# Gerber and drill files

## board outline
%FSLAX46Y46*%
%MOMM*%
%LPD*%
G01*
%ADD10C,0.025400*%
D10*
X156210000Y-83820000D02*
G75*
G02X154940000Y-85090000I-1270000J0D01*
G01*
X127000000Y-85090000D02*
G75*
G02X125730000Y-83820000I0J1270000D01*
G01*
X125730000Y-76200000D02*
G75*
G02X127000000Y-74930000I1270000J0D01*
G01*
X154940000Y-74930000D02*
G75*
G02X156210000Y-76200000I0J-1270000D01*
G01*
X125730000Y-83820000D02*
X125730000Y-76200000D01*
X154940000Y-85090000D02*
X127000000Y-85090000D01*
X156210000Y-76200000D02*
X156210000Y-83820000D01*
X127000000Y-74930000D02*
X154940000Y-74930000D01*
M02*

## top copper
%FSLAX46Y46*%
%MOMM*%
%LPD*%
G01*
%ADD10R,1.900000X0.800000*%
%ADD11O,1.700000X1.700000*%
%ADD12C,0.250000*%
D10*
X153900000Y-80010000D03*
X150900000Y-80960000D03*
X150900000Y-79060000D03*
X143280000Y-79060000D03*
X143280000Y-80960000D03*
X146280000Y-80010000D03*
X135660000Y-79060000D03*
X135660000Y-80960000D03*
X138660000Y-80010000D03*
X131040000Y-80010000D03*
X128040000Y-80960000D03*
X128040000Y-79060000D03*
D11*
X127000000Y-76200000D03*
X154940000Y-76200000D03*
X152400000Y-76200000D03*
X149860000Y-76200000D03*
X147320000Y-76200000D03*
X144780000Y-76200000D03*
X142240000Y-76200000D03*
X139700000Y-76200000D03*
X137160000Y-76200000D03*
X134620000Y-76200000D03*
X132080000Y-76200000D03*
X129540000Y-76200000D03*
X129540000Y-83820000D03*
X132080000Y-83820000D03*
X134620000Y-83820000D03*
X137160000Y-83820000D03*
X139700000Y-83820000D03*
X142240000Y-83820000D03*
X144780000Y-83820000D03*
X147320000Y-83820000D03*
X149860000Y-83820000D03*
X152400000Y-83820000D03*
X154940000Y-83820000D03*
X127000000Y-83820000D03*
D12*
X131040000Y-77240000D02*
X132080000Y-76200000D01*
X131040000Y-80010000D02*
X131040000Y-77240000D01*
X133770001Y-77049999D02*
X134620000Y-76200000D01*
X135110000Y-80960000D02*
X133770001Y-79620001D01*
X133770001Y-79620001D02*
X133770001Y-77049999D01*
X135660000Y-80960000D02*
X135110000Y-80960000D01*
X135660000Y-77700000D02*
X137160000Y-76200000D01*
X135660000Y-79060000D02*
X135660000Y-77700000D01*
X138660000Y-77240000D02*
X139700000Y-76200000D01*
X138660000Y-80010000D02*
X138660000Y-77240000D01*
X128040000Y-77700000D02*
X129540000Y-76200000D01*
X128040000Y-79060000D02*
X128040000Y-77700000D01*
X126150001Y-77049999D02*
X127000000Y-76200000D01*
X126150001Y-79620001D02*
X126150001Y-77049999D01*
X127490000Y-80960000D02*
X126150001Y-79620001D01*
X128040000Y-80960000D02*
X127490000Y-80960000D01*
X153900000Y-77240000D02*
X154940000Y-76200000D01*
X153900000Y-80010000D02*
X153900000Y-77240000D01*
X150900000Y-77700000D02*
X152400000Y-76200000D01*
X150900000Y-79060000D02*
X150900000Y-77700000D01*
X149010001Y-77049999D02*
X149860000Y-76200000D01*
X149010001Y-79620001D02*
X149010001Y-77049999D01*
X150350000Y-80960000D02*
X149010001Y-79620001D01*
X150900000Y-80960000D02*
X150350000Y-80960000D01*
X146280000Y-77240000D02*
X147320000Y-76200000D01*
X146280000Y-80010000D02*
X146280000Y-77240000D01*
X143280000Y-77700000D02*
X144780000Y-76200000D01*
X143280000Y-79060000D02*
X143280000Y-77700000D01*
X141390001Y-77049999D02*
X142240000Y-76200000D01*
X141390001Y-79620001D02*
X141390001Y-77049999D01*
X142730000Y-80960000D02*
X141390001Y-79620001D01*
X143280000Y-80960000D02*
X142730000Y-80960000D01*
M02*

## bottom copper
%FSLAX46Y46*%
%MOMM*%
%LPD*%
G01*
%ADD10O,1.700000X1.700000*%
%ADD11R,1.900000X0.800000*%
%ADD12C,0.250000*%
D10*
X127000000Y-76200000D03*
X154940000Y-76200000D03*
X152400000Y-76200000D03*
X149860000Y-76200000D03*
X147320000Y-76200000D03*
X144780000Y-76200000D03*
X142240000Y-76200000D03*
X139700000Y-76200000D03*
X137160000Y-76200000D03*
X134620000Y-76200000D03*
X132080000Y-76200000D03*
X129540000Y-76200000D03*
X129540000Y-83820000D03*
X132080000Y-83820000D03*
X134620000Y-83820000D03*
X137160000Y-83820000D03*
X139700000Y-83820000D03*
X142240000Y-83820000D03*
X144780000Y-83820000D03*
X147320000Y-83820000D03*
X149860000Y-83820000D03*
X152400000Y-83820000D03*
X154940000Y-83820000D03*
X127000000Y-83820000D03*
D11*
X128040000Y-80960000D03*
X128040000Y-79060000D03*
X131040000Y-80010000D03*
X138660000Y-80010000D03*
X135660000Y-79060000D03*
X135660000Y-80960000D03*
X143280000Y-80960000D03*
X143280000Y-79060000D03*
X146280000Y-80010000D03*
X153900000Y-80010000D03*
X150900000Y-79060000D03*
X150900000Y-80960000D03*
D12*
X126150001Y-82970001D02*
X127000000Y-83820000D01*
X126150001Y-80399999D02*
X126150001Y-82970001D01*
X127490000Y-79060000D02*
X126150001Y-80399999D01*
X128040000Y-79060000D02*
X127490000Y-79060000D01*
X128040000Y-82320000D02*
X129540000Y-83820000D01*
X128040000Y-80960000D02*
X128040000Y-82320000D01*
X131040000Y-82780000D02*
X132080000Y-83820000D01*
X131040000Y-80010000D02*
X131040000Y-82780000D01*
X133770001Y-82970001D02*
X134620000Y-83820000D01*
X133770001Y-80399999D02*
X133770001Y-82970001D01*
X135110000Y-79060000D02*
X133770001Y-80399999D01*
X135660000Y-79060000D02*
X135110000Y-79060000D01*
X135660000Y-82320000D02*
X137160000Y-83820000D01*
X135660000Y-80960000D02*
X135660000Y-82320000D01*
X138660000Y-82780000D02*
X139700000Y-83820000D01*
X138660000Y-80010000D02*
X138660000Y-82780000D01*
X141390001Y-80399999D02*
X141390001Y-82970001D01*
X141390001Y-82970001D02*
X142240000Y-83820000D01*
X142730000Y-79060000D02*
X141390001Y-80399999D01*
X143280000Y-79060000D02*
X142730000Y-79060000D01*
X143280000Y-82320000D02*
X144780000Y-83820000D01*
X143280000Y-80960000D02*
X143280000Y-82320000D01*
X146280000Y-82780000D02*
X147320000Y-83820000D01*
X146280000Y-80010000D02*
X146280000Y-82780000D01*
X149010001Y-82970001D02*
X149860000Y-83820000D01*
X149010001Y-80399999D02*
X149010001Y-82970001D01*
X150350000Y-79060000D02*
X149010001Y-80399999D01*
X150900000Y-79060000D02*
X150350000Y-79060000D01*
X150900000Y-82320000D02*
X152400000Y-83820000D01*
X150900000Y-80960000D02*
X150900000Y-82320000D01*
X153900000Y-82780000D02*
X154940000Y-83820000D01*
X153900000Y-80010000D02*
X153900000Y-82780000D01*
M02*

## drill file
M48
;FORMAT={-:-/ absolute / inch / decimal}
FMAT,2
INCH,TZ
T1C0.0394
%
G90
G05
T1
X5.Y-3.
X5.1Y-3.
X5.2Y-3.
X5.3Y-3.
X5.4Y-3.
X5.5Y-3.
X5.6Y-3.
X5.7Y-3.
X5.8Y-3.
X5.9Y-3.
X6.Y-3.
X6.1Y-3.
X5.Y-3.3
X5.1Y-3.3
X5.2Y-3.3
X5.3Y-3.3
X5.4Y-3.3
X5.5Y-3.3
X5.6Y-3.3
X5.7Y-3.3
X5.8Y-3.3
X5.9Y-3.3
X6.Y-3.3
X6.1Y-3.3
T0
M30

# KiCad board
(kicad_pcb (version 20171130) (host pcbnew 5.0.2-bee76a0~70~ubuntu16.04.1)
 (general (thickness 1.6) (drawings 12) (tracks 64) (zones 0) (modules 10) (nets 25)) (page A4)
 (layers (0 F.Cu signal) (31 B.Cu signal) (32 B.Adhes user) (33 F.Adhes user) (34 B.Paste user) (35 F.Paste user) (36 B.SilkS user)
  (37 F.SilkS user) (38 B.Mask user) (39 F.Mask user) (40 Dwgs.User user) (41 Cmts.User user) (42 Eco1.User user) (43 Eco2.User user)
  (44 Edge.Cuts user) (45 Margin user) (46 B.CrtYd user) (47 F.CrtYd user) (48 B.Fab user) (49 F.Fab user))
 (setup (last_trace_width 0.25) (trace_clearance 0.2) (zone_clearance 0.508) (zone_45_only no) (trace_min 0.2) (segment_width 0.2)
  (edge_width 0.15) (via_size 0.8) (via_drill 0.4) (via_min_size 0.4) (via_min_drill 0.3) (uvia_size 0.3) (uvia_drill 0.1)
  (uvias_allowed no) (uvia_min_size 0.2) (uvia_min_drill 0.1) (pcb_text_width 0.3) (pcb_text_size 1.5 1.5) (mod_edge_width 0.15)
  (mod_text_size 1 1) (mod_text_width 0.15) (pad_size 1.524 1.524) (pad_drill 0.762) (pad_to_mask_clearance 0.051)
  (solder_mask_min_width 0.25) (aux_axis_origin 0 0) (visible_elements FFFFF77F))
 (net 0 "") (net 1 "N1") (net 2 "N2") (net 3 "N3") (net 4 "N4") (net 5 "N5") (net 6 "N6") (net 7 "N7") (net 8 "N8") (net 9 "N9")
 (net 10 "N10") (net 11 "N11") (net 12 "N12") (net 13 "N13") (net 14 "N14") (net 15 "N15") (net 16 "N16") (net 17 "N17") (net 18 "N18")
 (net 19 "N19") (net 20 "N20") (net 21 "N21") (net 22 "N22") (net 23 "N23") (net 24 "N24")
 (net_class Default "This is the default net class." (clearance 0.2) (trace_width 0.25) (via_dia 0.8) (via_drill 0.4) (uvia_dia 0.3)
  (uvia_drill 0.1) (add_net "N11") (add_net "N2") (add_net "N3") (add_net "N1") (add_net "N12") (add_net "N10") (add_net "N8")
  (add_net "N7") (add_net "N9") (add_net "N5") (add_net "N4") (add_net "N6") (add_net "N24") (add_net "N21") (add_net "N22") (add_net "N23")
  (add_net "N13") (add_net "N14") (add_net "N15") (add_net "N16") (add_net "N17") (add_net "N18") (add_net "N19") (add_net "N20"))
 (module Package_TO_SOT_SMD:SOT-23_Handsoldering (layer F.Cu) (at 152.4 80.01)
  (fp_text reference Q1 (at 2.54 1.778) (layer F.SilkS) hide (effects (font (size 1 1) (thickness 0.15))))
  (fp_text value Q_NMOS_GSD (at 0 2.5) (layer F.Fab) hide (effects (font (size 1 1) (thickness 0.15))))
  (pad 3 smd rect (at 1.5 0) (size 1.9 0.8) (layers F.Cu F.Paste F.Mask) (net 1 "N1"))
  (pad 2 smd rect (at -1.5 0.95) (size 1.9 0.8) (layers F.Cu F.Paste F.Mask) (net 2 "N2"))
  (pad 1 smd rect (at -1.5 -0.95) (size 1.9 0.8) (layers F.Cu F.Paste F.Mask) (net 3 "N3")))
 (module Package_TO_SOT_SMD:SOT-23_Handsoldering (layer F.Cu) (at 144.78 80.01)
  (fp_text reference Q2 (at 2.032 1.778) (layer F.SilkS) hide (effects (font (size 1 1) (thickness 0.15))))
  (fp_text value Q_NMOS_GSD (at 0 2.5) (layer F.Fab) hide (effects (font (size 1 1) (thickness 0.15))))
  (pad 1 smd rect (at -1.5 -0.95) (size 1.9 0.8) (layers F.Cu F.Paste F.Mask) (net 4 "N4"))
  (pad 2 smd rect (at -1.5 0.95) (size 1.9 0.8) (layers F.Cu F.Paste F.Mask) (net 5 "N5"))
  (pad 3 smd rect (at 1.5 0) (size 1.9 0.8) (layers F.Cu F.Paste F.Mask) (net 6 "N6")))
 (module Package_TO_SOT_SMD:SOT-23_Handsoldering (layer F.Cu) (at 137.16 80.01)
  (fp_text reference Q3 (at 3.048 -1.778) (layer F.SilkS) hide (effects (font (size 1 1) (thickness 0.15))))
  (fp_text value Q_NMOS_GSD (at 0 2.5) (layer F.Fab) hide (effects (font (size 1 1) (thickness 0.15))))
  (pad 1 smd rect (at -1.5 -0.95) (size 1.9 0.8) (layers F.Cu F.Paste F.Mask) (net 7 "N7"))
  (pad 2 smd rect (at -1.5 0.95) (size 1.9 0.8) (layers F.Cu F.Paste F.Mask) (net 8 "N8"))
  (pad 3 smd rect (at 1.5 0) (size 1.9 0.8) (layers F.Cu F.Paste F.Mask) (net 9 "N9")))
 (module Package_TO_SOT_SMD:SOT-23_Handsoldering (layer F.Cu) (at 129.54 80.01)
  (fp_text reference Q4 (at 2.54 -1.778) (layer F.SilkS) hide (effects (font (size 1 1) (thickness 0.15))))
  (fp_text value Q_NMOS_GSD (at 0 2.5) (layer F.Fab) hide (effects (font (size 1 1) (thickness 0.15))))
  (pad 3 smd rect (at 1.5 0) (size 1.9 0.8) (layers F.Cu F.Paste F.Mask) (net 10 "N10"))
  (pad 2 smd rect (at -1.5 0.95) (size 1.9 0.8) (layers F.Cu F.Paste F.Mask) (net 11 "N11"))
  (pad 1 smd rect (at -1.5 -0.95) (size 1.9 0.8) (layers F.Cu F.Paste F.Mask) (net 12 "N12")))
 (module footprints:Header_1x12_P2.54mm (layer F.Cu) (at 127 76.2 90)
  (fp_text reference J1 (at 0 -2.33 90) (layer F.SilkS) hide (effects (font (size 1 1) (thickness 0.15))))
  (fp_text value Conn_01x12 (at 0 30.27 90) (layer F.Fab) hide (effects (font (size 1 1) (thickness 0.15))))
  (pad 1 thru_hole oval (at 0 0 90) (size 1.7 1.7) (drill 1) (layers *.Cu *.Mask) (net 11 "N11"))
  (pad 12 thru_hole oval (at 0 27.94 90) (size 1.7 1.7) (drill 1) (layers *.Cu *.Mask) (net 1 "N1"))
  (pad 11 thru_hole oval (at 0 25.4 90) (size 1.7 1.7) (drill 1) (layers *.Cu *.Mask) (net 3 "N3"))
  (pad 10 thru_hole oval (at 0 22.86 90) (size 1.7 1.7) (drill 1) (layers *.Cu *.Mask) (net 2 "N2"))
  (pad 9 thru_hole oval (at 0 20.32 90) (size 1.7 1.7) (drill 1) (layers *.Cu *.Mask) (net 6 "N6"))
  (pad 8 thru_hole oval (at 0 17.78 90) (size 1.7 1.7) (drill 1) (layers *.Cu *.Mask) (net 4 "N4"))
  (pad 7 thru_hole oval (at 0 15.24 90) (size 1.7 1.7) (drill 1) (layers *.Cu *.Mask) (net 5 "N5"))
  (pad 6 thru_hole oval (at 0 12.7 90) (size 1.7 1.7) (drill 1) (layers *.Cu *.Mask) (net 9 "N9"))
  (pad 5 thru_hole oval (at 0 10.16 90) (size 1.7 1.7) (drill 1) (layers *.Cu *.Mask) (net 7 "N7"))
  (pad 4 thru_hole oval (at 0 7.62 90) (size 1.7 1.7) (drill 1) (layers *.Cu *.Mask) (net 8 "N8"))
  (pad 3 thru_hole oval (at 0 5.08 90) (size 1.7 1.7) (drill 1) (layers *.Cu *.Mask) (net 10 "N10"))
  (pad 2 thru_hole oval (at 0 2.54 90) (size 1.7 1.7) (drill 1) (layers *.Cu *.Mask) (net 12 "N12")))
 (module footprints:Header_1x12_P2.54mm (layer F.Cu) (at 127 83.82 90)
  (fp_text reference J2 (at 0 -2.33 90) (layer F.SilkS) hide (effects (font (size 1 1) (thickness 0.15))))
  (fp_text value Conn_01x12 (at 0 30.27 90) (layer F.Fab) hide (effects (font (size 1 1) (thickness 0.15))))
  (pad 2 thru_hole oval (at 0 2.54 90) (size 1.7 1.7) (drill 1) (layers *.Cu *.Mask) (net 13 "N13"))
  (pad 3 thru_hole oval (at 0 5.08 90) (size 1.7 1.7) (drill 1) (layers *.Cu *.Mask) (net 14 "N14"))
  (pad 4 thru_hole oval (at 0 7.62 90) (size 1.7 1.7) (drill 1) (layers *.Cu *.Mask) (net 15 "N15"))
  (pad 5 thru_hole oval (at 0 10.16 90) (size 1.7 1.7) (drill 1) (layers *.Cu *.Mask) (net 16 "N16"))
  (pad 6 thru_hole oval (at 0 12.7 90) (size 1.7 1.7) (drill 1) (layers *.Cu *.Mask) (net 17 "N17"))
  (pad 7 thru_hole oval (at 0 15.24 90) (size 1.7 1.7) (drill 1) (layers *.Cu *.Mask) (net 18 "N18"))
  (pad 8 thru_hole oval (at 0 17.78 90) (size 1.7 1.7) (drill 1) (layers *.Cu *.Mask) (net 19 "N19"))
  (pad 9 thru_hole oval (at 0 20.32 90) (size 1.7 1.7) (drill 1) (layers *.Cu *.Mask) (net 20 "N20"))
  (pad 10 thru_hole oval (at 0 22.86 90) (size 1.7 1.7) (drill 1) (layers *.Cu *.Mask) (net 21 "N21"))
  (pad 11 thru_hole oval (at 0 25.4 90) (size 1.7 1.7) (drill 1) (layers *.Cu *.Mask) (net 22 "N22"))
  (pad 12 thru_hole oval (at 0 27.94 90) (size 1.7 1.7) (drill 1) (layers *.Cu *.Mask) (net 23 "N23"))
  (pad 1 thru_hole oval (at 0 0 90) (size 1.7 1.7) (drill 1) (layers *.Cu *.Mask) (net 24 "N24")))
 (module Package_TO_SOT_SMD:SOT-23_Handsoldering (layer B.Cu) (at 129.54 80.01)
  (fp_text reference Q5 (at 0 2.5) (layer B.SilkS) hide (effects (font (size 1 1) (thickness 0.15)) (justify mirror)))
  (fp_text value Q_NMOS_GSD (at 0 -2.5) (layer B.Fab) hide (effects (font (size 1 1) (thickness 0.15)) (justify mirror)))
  (pad 1 smd rect (at -1.5 0.95) (size 1.9 0.8) (layers B.Cu B.Paste B.Mask) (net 13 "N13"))
  (pad 2 smd rect (at -1.5 -0.95) (size 1.9 0.8) (layers B.Cu B.Paste B.Mask) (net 24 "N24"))
  (pad 3 smd rect (at 1.5 0) (size 1.9 0.8) (layers B.Cu B.Paste B.Mask) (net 14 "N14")))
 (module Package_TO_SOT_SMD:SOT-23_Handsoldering (layer B.Cu) (at 137.16 80.01)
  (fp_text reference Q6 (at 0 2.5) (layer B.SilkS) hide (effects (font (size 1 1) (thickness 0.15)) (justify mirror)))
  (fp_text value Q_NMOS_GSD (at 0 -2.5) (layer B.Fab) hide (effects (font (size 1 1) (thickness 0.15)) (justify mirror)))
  (pad 3 smd rect (at 1.5 0) (size 1.9 0.8) (layers B.Cu B.Paste B.Mask) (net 17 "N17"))
  (pad 2 smd rect (at -1.5 -0.95) (size 1.9 0.8) (layers B.Cu B.Paste B.Mask) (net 15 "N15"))
  (pad 1 smd rect (at -1.5 0.95) (size 1.9 0.8) (layers B.Cu B.Paste B.Mask) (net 16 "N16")))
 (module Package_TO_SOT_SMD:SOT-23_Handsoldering (layer B.Cu) (at 144.78 80.01)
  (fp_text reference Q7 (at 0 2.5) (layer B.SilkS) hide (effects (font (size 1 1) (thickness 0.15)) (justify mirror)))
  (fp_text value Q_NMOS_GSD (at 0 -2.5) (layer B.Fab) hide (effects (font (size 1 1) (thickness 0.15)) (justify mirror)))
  (pad 1 smd rect (at -1.5 0.95) (size 1.9 0.8) (layers B.Cu B.Paste B.Mask) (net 19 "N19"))
  (pad 2 smd rect (at -1.5 -0.95) (size 1.9 0.8) (layers B.Cu B.Paste B.Mask) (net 18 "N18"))
  (pad 3 smd rect (at 1.5 0) (size 1.9 0.8) (layers B.Cu B.Paste B.Mask) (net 20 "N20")))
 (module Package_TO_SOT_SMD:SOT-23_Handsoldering (layer B.Cu) (at 152.4 80.01)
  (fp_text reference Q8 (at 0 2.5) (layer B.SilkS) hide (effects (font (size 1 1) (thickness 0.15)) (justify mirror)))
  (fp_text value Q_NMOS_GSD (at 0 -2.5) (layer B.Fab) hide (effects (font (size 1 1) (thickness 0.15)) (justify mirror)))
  (pad 3 smd rect (at 1.5 0) (size 1.9 0.8) (layers B.Cu B.Paste B.Mask) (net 23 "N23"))
  (pad 2 smd rect (at -1.5 -0.95) (size 1.9 0.8) (layers B.Cu B.Paste B.Mask) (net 21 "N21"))
  (pad 1 smd rect (at -1.5 0.95) (size 1.9 0.8) (layers B.Cu B.Paste B.Mask) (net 22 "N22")))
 (gr_arc (start 154.94 83.82) (end 154.94 85.09) (angle -90) (layer Edge.Cuts) (width 0.0254))
 (gr_arc (start 127 83.82) (end 125.73 83.82) (angle -90) (layer Edge.Cuts) (width 0.0254))
 (gr_arc (start 127 76.2) (end 127 74.93) (angle -90) (layer Edge.Cuts) (width 0.0254))
 (gr_arc (start 154.94 76.2) (end 156.21 76.2) (angle -90) (layer Edge.Cuts) (width 0.0254))
 (gr_line (start 125.73 83.82) (end 125.73 76.2) (layer Edge.Cuts) (width 0.0254))
 (gr_line (start 154.94 85.09) (end 127 85.09) (layer Edge.Cuts) (width 0.0254))
 (gr_line (start 156.21 76.2) (end 156.21 83.82) (layer Edge.Cuts) (width 0.0254))
 (gr_line (start 127 74.93) (end 154.94 74.93) (layer Edge.Cuts) (width 0.0254))
 (segment (start 131.04 77.24) (end 132.08 76.2) (width 0.25) (layer F.Cu) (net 10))
 (segment (start 131.04 80.01) (end 131.04 77.24) (width 0.25) (layer F.Cu) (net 10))
 (segment (start 133.770001 77.049999) (end 134.62 76.2) (width 0.25) (layer F.Cu) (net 8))
 (segment (start 135.11 80.96) (end 133.770001 79.620001) (width 0.25) (layer F.Cu) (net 8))
 (segment (start 133.770001 79.620001) (end 133.770001 77.049999) (width 0.25) (layer F.Cu) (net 8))
 (segment (start 135.66 80.96) (end 135.11 80.96) (width 0.25) (layer F.Cu) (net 8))
 (segment (start 135.66 77.7) (end 137.16 76.2) (width 0.25) (layer F.Cu) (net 7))
 (segment (start 135.66 79.06) (end 135.66 77.7) (width 0.25) (layer F.Cu) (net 7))
 (segment (start 138.66 77.24) (end 139.7 76.2) (width 0.25) (layer F.Cu) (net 9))
 (segment (start 138.66 80.01) (end 138.66 77.24) (width 0.25) (layer F.Cu) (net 9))
 (segment (start 128.04 77.7) (end 129.54 76.2) (width 0.25) (layer F.Cu) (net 12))
 (segment (start 128.04 79.06) (end 128.04 77.7) (width 0.25) (layer F.Cu) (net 12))
 (segment (start 126.150001 77.049999) (end 127 76.2) (width 0.25) (layer F.Cu) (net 11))
 (segment (start 126.150001 79.620001) (end 126.150001 77.049999) (width 0.25) (layer F.Cu) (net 11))
 (segment (start 127.49 80.96) (end 126.150001 79.620001) (width 0.25) (layer F.Cu) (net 11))
 (segment (start 128.04 80.96) (end 127.49 80.96) (width 0.25) (layer F.Cu) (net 11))
 (segment (start 126.150001 82.970001) (end 127 83.82) (width 0.25) (layer B.Cu) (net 24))
 (segment (start 126.150001 80.399999) (end 126.150001 82.970001) (width 0.25) (layer B.Cu) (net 24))
 (segment (start 127.49 79.06) (end 126.150001 80.399999) (width 0.25) (layer B.Cu) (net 24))
 (segment (start 128.04 79.06) (end 127.49 79.06) (width 0.25) (layer B.Cu) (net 24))
 (segment (start 128.04 82.32) (end 129.54 83.82) (width 0.25) (layer B.Cu) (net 13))
 (segment (start 128.04 80.96) (end 128.04 82.32) (width 0.25) (layer B.Cu) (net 13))
 (segment (start 131.04 82.78) (end 132.08 83.82) (width 0.25) (layer B.Cu) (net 14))
 (segment (start 131.04 80.01) (end 131.04 82.78) (width 0.25) (layer B.Cu) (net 14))
 (segment (start 133.770001 82.970001) (end 134.62 83.82) (width 0.25) (layer B.Cu) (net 15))
 (segment (start 133.770001 80.399999) (end 133.770001 82.970001) (width 0.25) (layer B.Cu) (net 15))
 (segment (start 135.11 79.06) (end 133.770001 80.399999) (width 0.25) (layer B.Cu) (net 15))
 (segment (start 135.66 79.06) (end 135.11 79.06) (width 0.25) (layer B.Cu) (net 15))
 (segment (start 135.66 82.32) (end 137.16 83.82) (width 0.25) (layer B.Cu) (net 16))
 (segment (start 135.66 80.96) (end 135.66 82.32) (width 0.25) (layer B.Cu) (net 16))
 (segment (start 138.66 82.78) (end 139.7 83.82) (width 0.25) (layer B.Cu) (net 17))
 (segment (start 138.66 80.01) (end 138.66 82.78) (width 0.25) (layer B.Cu) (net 17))
 (segment (start 153.9 77.24) (end 154.94 76.2) (width 0.25) (layer F.Cu) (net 1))
 (segment (start 153.9 80.01) (end 153.9 77.24) (width 0.25) (layer F.Cu) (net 1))
 (segment (start 150.9 77.7) (end 152.4 76.2) (width 0.25) (layer F.Cu) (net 3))
 (segment (start 150.9 79.06) (end 150.9 77.7) (width 0.25) (layer F.Cu) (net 3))
 (segment (start 149.010001 77.049999) (end 149.86 76.2) (width 0.25) (layer F.Cu) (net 2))
 (segment (start 149.010001 79.620001) (end 149.010001 77.049999) (width 0.25) (layer F.Cu) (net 2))
 (segment (start 150.35 80.96) (end 149.010001 79.620001) (width 0.25) (layer F.Cu) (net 2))
 (segment (start 150.9 80.96) (end 150.35 80.96) (width 0.25) (layer F.Cu) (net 2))
 (segment (start 146.28 77.24) (end 147.32 76.2) (width 0.25) (layer F.Cu) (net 6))
 (segment (start 146.28 80.01) (end 146.28 77.24) (width 0.25) (layer F.Cu) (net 6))
 (segment (start 143.28 77.7) (end 144.78 76.2) (width 0.25) (layer F.Cu) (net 4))
 (segment (start 143.28 79.06) (end 143.28 77.7) (width 0.25) (layer F.Cu) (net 4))
 (segment (start 141.390001 77.049999) (end 142.24 76.2) (width 0.25) (layer F.Cu) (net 5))
 (segment (start 141.390001 79.620001) (end 141.390001 77.049999) (width 0.25) (layer F.Cu) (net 5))
 (segment (start 142.73 80.96) (end 141.390001 79.620001) (width 0.25) (layer F.Cu) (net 5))
 (segment (start 143.28 80.96) (end 142.73 80.96) (width 0.25) (layer F.Cu) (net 5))
 (segment (start 141.390001 80.399999) (end 141.390001 82.970001) (width 0.25) (layer B.Cu) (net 18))
 (segment (start 141.390001 82.970001) (end 142.24 83.82) (width 0.25) (layer B.Cu) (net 18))
 (segment (start 142.73 79.06) (end 141.390001 80.399999) (width 0.25) (layer B.Cu) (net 18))
 (segment (start 143.28 79.06) (end 142.73 79.06) (width 0.25) (layer B.Cu) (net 18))
 (segment (start 143.28 82.32) (end 144.78 83.82) (width 0.25) (layer B.Cu) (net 19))
 (segment (start 143.28 80.96) (end 143.28 82.32) (width 0.25) (layer B.Cu) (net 19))
 (segment (start 146.28 82.78) (end 147.32 83.82) (width 0.25) (layer B.Cu) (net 20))
 (segment (start 146.28 80.01) (end 146.28 82.78) (width 0.25) (layer B.Cu) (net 20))
 (segment (start 149.010001 82.970001) (end 149.86 83.82) (width 0.25) (layer B.Cu) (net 21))
 (segment (start 149.010001 80.399999) (end 149.010001 82.970001) (width 0.25) (layer B.Cu) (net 21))
 (segment (start 150.35 79.06) (end 149.010001 80.399999) (width 0.25) (layer B.Cu) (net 21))
 (segment (start 150.9 79.06) (end 150.35 79.06) (width 0.25) (layer B.Cu) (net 21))
 (segment (start 150.9 82.32) (end 152.4 83.82) (width 0.25) (layer B.Cu) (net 22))
 (segment (start 150.9 80.96) (end 150.9 82.32) (width 0.25) (layer B.Cu) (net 22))
 (segment (start 153.9 82.78) (end 154.94 83.82) (width 0.25) (layer B.Cu) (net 23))
 (segment (start 153.9 80.01) (end 153.9 82.78) (width 0.25) (layer B.Cu) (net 23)))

